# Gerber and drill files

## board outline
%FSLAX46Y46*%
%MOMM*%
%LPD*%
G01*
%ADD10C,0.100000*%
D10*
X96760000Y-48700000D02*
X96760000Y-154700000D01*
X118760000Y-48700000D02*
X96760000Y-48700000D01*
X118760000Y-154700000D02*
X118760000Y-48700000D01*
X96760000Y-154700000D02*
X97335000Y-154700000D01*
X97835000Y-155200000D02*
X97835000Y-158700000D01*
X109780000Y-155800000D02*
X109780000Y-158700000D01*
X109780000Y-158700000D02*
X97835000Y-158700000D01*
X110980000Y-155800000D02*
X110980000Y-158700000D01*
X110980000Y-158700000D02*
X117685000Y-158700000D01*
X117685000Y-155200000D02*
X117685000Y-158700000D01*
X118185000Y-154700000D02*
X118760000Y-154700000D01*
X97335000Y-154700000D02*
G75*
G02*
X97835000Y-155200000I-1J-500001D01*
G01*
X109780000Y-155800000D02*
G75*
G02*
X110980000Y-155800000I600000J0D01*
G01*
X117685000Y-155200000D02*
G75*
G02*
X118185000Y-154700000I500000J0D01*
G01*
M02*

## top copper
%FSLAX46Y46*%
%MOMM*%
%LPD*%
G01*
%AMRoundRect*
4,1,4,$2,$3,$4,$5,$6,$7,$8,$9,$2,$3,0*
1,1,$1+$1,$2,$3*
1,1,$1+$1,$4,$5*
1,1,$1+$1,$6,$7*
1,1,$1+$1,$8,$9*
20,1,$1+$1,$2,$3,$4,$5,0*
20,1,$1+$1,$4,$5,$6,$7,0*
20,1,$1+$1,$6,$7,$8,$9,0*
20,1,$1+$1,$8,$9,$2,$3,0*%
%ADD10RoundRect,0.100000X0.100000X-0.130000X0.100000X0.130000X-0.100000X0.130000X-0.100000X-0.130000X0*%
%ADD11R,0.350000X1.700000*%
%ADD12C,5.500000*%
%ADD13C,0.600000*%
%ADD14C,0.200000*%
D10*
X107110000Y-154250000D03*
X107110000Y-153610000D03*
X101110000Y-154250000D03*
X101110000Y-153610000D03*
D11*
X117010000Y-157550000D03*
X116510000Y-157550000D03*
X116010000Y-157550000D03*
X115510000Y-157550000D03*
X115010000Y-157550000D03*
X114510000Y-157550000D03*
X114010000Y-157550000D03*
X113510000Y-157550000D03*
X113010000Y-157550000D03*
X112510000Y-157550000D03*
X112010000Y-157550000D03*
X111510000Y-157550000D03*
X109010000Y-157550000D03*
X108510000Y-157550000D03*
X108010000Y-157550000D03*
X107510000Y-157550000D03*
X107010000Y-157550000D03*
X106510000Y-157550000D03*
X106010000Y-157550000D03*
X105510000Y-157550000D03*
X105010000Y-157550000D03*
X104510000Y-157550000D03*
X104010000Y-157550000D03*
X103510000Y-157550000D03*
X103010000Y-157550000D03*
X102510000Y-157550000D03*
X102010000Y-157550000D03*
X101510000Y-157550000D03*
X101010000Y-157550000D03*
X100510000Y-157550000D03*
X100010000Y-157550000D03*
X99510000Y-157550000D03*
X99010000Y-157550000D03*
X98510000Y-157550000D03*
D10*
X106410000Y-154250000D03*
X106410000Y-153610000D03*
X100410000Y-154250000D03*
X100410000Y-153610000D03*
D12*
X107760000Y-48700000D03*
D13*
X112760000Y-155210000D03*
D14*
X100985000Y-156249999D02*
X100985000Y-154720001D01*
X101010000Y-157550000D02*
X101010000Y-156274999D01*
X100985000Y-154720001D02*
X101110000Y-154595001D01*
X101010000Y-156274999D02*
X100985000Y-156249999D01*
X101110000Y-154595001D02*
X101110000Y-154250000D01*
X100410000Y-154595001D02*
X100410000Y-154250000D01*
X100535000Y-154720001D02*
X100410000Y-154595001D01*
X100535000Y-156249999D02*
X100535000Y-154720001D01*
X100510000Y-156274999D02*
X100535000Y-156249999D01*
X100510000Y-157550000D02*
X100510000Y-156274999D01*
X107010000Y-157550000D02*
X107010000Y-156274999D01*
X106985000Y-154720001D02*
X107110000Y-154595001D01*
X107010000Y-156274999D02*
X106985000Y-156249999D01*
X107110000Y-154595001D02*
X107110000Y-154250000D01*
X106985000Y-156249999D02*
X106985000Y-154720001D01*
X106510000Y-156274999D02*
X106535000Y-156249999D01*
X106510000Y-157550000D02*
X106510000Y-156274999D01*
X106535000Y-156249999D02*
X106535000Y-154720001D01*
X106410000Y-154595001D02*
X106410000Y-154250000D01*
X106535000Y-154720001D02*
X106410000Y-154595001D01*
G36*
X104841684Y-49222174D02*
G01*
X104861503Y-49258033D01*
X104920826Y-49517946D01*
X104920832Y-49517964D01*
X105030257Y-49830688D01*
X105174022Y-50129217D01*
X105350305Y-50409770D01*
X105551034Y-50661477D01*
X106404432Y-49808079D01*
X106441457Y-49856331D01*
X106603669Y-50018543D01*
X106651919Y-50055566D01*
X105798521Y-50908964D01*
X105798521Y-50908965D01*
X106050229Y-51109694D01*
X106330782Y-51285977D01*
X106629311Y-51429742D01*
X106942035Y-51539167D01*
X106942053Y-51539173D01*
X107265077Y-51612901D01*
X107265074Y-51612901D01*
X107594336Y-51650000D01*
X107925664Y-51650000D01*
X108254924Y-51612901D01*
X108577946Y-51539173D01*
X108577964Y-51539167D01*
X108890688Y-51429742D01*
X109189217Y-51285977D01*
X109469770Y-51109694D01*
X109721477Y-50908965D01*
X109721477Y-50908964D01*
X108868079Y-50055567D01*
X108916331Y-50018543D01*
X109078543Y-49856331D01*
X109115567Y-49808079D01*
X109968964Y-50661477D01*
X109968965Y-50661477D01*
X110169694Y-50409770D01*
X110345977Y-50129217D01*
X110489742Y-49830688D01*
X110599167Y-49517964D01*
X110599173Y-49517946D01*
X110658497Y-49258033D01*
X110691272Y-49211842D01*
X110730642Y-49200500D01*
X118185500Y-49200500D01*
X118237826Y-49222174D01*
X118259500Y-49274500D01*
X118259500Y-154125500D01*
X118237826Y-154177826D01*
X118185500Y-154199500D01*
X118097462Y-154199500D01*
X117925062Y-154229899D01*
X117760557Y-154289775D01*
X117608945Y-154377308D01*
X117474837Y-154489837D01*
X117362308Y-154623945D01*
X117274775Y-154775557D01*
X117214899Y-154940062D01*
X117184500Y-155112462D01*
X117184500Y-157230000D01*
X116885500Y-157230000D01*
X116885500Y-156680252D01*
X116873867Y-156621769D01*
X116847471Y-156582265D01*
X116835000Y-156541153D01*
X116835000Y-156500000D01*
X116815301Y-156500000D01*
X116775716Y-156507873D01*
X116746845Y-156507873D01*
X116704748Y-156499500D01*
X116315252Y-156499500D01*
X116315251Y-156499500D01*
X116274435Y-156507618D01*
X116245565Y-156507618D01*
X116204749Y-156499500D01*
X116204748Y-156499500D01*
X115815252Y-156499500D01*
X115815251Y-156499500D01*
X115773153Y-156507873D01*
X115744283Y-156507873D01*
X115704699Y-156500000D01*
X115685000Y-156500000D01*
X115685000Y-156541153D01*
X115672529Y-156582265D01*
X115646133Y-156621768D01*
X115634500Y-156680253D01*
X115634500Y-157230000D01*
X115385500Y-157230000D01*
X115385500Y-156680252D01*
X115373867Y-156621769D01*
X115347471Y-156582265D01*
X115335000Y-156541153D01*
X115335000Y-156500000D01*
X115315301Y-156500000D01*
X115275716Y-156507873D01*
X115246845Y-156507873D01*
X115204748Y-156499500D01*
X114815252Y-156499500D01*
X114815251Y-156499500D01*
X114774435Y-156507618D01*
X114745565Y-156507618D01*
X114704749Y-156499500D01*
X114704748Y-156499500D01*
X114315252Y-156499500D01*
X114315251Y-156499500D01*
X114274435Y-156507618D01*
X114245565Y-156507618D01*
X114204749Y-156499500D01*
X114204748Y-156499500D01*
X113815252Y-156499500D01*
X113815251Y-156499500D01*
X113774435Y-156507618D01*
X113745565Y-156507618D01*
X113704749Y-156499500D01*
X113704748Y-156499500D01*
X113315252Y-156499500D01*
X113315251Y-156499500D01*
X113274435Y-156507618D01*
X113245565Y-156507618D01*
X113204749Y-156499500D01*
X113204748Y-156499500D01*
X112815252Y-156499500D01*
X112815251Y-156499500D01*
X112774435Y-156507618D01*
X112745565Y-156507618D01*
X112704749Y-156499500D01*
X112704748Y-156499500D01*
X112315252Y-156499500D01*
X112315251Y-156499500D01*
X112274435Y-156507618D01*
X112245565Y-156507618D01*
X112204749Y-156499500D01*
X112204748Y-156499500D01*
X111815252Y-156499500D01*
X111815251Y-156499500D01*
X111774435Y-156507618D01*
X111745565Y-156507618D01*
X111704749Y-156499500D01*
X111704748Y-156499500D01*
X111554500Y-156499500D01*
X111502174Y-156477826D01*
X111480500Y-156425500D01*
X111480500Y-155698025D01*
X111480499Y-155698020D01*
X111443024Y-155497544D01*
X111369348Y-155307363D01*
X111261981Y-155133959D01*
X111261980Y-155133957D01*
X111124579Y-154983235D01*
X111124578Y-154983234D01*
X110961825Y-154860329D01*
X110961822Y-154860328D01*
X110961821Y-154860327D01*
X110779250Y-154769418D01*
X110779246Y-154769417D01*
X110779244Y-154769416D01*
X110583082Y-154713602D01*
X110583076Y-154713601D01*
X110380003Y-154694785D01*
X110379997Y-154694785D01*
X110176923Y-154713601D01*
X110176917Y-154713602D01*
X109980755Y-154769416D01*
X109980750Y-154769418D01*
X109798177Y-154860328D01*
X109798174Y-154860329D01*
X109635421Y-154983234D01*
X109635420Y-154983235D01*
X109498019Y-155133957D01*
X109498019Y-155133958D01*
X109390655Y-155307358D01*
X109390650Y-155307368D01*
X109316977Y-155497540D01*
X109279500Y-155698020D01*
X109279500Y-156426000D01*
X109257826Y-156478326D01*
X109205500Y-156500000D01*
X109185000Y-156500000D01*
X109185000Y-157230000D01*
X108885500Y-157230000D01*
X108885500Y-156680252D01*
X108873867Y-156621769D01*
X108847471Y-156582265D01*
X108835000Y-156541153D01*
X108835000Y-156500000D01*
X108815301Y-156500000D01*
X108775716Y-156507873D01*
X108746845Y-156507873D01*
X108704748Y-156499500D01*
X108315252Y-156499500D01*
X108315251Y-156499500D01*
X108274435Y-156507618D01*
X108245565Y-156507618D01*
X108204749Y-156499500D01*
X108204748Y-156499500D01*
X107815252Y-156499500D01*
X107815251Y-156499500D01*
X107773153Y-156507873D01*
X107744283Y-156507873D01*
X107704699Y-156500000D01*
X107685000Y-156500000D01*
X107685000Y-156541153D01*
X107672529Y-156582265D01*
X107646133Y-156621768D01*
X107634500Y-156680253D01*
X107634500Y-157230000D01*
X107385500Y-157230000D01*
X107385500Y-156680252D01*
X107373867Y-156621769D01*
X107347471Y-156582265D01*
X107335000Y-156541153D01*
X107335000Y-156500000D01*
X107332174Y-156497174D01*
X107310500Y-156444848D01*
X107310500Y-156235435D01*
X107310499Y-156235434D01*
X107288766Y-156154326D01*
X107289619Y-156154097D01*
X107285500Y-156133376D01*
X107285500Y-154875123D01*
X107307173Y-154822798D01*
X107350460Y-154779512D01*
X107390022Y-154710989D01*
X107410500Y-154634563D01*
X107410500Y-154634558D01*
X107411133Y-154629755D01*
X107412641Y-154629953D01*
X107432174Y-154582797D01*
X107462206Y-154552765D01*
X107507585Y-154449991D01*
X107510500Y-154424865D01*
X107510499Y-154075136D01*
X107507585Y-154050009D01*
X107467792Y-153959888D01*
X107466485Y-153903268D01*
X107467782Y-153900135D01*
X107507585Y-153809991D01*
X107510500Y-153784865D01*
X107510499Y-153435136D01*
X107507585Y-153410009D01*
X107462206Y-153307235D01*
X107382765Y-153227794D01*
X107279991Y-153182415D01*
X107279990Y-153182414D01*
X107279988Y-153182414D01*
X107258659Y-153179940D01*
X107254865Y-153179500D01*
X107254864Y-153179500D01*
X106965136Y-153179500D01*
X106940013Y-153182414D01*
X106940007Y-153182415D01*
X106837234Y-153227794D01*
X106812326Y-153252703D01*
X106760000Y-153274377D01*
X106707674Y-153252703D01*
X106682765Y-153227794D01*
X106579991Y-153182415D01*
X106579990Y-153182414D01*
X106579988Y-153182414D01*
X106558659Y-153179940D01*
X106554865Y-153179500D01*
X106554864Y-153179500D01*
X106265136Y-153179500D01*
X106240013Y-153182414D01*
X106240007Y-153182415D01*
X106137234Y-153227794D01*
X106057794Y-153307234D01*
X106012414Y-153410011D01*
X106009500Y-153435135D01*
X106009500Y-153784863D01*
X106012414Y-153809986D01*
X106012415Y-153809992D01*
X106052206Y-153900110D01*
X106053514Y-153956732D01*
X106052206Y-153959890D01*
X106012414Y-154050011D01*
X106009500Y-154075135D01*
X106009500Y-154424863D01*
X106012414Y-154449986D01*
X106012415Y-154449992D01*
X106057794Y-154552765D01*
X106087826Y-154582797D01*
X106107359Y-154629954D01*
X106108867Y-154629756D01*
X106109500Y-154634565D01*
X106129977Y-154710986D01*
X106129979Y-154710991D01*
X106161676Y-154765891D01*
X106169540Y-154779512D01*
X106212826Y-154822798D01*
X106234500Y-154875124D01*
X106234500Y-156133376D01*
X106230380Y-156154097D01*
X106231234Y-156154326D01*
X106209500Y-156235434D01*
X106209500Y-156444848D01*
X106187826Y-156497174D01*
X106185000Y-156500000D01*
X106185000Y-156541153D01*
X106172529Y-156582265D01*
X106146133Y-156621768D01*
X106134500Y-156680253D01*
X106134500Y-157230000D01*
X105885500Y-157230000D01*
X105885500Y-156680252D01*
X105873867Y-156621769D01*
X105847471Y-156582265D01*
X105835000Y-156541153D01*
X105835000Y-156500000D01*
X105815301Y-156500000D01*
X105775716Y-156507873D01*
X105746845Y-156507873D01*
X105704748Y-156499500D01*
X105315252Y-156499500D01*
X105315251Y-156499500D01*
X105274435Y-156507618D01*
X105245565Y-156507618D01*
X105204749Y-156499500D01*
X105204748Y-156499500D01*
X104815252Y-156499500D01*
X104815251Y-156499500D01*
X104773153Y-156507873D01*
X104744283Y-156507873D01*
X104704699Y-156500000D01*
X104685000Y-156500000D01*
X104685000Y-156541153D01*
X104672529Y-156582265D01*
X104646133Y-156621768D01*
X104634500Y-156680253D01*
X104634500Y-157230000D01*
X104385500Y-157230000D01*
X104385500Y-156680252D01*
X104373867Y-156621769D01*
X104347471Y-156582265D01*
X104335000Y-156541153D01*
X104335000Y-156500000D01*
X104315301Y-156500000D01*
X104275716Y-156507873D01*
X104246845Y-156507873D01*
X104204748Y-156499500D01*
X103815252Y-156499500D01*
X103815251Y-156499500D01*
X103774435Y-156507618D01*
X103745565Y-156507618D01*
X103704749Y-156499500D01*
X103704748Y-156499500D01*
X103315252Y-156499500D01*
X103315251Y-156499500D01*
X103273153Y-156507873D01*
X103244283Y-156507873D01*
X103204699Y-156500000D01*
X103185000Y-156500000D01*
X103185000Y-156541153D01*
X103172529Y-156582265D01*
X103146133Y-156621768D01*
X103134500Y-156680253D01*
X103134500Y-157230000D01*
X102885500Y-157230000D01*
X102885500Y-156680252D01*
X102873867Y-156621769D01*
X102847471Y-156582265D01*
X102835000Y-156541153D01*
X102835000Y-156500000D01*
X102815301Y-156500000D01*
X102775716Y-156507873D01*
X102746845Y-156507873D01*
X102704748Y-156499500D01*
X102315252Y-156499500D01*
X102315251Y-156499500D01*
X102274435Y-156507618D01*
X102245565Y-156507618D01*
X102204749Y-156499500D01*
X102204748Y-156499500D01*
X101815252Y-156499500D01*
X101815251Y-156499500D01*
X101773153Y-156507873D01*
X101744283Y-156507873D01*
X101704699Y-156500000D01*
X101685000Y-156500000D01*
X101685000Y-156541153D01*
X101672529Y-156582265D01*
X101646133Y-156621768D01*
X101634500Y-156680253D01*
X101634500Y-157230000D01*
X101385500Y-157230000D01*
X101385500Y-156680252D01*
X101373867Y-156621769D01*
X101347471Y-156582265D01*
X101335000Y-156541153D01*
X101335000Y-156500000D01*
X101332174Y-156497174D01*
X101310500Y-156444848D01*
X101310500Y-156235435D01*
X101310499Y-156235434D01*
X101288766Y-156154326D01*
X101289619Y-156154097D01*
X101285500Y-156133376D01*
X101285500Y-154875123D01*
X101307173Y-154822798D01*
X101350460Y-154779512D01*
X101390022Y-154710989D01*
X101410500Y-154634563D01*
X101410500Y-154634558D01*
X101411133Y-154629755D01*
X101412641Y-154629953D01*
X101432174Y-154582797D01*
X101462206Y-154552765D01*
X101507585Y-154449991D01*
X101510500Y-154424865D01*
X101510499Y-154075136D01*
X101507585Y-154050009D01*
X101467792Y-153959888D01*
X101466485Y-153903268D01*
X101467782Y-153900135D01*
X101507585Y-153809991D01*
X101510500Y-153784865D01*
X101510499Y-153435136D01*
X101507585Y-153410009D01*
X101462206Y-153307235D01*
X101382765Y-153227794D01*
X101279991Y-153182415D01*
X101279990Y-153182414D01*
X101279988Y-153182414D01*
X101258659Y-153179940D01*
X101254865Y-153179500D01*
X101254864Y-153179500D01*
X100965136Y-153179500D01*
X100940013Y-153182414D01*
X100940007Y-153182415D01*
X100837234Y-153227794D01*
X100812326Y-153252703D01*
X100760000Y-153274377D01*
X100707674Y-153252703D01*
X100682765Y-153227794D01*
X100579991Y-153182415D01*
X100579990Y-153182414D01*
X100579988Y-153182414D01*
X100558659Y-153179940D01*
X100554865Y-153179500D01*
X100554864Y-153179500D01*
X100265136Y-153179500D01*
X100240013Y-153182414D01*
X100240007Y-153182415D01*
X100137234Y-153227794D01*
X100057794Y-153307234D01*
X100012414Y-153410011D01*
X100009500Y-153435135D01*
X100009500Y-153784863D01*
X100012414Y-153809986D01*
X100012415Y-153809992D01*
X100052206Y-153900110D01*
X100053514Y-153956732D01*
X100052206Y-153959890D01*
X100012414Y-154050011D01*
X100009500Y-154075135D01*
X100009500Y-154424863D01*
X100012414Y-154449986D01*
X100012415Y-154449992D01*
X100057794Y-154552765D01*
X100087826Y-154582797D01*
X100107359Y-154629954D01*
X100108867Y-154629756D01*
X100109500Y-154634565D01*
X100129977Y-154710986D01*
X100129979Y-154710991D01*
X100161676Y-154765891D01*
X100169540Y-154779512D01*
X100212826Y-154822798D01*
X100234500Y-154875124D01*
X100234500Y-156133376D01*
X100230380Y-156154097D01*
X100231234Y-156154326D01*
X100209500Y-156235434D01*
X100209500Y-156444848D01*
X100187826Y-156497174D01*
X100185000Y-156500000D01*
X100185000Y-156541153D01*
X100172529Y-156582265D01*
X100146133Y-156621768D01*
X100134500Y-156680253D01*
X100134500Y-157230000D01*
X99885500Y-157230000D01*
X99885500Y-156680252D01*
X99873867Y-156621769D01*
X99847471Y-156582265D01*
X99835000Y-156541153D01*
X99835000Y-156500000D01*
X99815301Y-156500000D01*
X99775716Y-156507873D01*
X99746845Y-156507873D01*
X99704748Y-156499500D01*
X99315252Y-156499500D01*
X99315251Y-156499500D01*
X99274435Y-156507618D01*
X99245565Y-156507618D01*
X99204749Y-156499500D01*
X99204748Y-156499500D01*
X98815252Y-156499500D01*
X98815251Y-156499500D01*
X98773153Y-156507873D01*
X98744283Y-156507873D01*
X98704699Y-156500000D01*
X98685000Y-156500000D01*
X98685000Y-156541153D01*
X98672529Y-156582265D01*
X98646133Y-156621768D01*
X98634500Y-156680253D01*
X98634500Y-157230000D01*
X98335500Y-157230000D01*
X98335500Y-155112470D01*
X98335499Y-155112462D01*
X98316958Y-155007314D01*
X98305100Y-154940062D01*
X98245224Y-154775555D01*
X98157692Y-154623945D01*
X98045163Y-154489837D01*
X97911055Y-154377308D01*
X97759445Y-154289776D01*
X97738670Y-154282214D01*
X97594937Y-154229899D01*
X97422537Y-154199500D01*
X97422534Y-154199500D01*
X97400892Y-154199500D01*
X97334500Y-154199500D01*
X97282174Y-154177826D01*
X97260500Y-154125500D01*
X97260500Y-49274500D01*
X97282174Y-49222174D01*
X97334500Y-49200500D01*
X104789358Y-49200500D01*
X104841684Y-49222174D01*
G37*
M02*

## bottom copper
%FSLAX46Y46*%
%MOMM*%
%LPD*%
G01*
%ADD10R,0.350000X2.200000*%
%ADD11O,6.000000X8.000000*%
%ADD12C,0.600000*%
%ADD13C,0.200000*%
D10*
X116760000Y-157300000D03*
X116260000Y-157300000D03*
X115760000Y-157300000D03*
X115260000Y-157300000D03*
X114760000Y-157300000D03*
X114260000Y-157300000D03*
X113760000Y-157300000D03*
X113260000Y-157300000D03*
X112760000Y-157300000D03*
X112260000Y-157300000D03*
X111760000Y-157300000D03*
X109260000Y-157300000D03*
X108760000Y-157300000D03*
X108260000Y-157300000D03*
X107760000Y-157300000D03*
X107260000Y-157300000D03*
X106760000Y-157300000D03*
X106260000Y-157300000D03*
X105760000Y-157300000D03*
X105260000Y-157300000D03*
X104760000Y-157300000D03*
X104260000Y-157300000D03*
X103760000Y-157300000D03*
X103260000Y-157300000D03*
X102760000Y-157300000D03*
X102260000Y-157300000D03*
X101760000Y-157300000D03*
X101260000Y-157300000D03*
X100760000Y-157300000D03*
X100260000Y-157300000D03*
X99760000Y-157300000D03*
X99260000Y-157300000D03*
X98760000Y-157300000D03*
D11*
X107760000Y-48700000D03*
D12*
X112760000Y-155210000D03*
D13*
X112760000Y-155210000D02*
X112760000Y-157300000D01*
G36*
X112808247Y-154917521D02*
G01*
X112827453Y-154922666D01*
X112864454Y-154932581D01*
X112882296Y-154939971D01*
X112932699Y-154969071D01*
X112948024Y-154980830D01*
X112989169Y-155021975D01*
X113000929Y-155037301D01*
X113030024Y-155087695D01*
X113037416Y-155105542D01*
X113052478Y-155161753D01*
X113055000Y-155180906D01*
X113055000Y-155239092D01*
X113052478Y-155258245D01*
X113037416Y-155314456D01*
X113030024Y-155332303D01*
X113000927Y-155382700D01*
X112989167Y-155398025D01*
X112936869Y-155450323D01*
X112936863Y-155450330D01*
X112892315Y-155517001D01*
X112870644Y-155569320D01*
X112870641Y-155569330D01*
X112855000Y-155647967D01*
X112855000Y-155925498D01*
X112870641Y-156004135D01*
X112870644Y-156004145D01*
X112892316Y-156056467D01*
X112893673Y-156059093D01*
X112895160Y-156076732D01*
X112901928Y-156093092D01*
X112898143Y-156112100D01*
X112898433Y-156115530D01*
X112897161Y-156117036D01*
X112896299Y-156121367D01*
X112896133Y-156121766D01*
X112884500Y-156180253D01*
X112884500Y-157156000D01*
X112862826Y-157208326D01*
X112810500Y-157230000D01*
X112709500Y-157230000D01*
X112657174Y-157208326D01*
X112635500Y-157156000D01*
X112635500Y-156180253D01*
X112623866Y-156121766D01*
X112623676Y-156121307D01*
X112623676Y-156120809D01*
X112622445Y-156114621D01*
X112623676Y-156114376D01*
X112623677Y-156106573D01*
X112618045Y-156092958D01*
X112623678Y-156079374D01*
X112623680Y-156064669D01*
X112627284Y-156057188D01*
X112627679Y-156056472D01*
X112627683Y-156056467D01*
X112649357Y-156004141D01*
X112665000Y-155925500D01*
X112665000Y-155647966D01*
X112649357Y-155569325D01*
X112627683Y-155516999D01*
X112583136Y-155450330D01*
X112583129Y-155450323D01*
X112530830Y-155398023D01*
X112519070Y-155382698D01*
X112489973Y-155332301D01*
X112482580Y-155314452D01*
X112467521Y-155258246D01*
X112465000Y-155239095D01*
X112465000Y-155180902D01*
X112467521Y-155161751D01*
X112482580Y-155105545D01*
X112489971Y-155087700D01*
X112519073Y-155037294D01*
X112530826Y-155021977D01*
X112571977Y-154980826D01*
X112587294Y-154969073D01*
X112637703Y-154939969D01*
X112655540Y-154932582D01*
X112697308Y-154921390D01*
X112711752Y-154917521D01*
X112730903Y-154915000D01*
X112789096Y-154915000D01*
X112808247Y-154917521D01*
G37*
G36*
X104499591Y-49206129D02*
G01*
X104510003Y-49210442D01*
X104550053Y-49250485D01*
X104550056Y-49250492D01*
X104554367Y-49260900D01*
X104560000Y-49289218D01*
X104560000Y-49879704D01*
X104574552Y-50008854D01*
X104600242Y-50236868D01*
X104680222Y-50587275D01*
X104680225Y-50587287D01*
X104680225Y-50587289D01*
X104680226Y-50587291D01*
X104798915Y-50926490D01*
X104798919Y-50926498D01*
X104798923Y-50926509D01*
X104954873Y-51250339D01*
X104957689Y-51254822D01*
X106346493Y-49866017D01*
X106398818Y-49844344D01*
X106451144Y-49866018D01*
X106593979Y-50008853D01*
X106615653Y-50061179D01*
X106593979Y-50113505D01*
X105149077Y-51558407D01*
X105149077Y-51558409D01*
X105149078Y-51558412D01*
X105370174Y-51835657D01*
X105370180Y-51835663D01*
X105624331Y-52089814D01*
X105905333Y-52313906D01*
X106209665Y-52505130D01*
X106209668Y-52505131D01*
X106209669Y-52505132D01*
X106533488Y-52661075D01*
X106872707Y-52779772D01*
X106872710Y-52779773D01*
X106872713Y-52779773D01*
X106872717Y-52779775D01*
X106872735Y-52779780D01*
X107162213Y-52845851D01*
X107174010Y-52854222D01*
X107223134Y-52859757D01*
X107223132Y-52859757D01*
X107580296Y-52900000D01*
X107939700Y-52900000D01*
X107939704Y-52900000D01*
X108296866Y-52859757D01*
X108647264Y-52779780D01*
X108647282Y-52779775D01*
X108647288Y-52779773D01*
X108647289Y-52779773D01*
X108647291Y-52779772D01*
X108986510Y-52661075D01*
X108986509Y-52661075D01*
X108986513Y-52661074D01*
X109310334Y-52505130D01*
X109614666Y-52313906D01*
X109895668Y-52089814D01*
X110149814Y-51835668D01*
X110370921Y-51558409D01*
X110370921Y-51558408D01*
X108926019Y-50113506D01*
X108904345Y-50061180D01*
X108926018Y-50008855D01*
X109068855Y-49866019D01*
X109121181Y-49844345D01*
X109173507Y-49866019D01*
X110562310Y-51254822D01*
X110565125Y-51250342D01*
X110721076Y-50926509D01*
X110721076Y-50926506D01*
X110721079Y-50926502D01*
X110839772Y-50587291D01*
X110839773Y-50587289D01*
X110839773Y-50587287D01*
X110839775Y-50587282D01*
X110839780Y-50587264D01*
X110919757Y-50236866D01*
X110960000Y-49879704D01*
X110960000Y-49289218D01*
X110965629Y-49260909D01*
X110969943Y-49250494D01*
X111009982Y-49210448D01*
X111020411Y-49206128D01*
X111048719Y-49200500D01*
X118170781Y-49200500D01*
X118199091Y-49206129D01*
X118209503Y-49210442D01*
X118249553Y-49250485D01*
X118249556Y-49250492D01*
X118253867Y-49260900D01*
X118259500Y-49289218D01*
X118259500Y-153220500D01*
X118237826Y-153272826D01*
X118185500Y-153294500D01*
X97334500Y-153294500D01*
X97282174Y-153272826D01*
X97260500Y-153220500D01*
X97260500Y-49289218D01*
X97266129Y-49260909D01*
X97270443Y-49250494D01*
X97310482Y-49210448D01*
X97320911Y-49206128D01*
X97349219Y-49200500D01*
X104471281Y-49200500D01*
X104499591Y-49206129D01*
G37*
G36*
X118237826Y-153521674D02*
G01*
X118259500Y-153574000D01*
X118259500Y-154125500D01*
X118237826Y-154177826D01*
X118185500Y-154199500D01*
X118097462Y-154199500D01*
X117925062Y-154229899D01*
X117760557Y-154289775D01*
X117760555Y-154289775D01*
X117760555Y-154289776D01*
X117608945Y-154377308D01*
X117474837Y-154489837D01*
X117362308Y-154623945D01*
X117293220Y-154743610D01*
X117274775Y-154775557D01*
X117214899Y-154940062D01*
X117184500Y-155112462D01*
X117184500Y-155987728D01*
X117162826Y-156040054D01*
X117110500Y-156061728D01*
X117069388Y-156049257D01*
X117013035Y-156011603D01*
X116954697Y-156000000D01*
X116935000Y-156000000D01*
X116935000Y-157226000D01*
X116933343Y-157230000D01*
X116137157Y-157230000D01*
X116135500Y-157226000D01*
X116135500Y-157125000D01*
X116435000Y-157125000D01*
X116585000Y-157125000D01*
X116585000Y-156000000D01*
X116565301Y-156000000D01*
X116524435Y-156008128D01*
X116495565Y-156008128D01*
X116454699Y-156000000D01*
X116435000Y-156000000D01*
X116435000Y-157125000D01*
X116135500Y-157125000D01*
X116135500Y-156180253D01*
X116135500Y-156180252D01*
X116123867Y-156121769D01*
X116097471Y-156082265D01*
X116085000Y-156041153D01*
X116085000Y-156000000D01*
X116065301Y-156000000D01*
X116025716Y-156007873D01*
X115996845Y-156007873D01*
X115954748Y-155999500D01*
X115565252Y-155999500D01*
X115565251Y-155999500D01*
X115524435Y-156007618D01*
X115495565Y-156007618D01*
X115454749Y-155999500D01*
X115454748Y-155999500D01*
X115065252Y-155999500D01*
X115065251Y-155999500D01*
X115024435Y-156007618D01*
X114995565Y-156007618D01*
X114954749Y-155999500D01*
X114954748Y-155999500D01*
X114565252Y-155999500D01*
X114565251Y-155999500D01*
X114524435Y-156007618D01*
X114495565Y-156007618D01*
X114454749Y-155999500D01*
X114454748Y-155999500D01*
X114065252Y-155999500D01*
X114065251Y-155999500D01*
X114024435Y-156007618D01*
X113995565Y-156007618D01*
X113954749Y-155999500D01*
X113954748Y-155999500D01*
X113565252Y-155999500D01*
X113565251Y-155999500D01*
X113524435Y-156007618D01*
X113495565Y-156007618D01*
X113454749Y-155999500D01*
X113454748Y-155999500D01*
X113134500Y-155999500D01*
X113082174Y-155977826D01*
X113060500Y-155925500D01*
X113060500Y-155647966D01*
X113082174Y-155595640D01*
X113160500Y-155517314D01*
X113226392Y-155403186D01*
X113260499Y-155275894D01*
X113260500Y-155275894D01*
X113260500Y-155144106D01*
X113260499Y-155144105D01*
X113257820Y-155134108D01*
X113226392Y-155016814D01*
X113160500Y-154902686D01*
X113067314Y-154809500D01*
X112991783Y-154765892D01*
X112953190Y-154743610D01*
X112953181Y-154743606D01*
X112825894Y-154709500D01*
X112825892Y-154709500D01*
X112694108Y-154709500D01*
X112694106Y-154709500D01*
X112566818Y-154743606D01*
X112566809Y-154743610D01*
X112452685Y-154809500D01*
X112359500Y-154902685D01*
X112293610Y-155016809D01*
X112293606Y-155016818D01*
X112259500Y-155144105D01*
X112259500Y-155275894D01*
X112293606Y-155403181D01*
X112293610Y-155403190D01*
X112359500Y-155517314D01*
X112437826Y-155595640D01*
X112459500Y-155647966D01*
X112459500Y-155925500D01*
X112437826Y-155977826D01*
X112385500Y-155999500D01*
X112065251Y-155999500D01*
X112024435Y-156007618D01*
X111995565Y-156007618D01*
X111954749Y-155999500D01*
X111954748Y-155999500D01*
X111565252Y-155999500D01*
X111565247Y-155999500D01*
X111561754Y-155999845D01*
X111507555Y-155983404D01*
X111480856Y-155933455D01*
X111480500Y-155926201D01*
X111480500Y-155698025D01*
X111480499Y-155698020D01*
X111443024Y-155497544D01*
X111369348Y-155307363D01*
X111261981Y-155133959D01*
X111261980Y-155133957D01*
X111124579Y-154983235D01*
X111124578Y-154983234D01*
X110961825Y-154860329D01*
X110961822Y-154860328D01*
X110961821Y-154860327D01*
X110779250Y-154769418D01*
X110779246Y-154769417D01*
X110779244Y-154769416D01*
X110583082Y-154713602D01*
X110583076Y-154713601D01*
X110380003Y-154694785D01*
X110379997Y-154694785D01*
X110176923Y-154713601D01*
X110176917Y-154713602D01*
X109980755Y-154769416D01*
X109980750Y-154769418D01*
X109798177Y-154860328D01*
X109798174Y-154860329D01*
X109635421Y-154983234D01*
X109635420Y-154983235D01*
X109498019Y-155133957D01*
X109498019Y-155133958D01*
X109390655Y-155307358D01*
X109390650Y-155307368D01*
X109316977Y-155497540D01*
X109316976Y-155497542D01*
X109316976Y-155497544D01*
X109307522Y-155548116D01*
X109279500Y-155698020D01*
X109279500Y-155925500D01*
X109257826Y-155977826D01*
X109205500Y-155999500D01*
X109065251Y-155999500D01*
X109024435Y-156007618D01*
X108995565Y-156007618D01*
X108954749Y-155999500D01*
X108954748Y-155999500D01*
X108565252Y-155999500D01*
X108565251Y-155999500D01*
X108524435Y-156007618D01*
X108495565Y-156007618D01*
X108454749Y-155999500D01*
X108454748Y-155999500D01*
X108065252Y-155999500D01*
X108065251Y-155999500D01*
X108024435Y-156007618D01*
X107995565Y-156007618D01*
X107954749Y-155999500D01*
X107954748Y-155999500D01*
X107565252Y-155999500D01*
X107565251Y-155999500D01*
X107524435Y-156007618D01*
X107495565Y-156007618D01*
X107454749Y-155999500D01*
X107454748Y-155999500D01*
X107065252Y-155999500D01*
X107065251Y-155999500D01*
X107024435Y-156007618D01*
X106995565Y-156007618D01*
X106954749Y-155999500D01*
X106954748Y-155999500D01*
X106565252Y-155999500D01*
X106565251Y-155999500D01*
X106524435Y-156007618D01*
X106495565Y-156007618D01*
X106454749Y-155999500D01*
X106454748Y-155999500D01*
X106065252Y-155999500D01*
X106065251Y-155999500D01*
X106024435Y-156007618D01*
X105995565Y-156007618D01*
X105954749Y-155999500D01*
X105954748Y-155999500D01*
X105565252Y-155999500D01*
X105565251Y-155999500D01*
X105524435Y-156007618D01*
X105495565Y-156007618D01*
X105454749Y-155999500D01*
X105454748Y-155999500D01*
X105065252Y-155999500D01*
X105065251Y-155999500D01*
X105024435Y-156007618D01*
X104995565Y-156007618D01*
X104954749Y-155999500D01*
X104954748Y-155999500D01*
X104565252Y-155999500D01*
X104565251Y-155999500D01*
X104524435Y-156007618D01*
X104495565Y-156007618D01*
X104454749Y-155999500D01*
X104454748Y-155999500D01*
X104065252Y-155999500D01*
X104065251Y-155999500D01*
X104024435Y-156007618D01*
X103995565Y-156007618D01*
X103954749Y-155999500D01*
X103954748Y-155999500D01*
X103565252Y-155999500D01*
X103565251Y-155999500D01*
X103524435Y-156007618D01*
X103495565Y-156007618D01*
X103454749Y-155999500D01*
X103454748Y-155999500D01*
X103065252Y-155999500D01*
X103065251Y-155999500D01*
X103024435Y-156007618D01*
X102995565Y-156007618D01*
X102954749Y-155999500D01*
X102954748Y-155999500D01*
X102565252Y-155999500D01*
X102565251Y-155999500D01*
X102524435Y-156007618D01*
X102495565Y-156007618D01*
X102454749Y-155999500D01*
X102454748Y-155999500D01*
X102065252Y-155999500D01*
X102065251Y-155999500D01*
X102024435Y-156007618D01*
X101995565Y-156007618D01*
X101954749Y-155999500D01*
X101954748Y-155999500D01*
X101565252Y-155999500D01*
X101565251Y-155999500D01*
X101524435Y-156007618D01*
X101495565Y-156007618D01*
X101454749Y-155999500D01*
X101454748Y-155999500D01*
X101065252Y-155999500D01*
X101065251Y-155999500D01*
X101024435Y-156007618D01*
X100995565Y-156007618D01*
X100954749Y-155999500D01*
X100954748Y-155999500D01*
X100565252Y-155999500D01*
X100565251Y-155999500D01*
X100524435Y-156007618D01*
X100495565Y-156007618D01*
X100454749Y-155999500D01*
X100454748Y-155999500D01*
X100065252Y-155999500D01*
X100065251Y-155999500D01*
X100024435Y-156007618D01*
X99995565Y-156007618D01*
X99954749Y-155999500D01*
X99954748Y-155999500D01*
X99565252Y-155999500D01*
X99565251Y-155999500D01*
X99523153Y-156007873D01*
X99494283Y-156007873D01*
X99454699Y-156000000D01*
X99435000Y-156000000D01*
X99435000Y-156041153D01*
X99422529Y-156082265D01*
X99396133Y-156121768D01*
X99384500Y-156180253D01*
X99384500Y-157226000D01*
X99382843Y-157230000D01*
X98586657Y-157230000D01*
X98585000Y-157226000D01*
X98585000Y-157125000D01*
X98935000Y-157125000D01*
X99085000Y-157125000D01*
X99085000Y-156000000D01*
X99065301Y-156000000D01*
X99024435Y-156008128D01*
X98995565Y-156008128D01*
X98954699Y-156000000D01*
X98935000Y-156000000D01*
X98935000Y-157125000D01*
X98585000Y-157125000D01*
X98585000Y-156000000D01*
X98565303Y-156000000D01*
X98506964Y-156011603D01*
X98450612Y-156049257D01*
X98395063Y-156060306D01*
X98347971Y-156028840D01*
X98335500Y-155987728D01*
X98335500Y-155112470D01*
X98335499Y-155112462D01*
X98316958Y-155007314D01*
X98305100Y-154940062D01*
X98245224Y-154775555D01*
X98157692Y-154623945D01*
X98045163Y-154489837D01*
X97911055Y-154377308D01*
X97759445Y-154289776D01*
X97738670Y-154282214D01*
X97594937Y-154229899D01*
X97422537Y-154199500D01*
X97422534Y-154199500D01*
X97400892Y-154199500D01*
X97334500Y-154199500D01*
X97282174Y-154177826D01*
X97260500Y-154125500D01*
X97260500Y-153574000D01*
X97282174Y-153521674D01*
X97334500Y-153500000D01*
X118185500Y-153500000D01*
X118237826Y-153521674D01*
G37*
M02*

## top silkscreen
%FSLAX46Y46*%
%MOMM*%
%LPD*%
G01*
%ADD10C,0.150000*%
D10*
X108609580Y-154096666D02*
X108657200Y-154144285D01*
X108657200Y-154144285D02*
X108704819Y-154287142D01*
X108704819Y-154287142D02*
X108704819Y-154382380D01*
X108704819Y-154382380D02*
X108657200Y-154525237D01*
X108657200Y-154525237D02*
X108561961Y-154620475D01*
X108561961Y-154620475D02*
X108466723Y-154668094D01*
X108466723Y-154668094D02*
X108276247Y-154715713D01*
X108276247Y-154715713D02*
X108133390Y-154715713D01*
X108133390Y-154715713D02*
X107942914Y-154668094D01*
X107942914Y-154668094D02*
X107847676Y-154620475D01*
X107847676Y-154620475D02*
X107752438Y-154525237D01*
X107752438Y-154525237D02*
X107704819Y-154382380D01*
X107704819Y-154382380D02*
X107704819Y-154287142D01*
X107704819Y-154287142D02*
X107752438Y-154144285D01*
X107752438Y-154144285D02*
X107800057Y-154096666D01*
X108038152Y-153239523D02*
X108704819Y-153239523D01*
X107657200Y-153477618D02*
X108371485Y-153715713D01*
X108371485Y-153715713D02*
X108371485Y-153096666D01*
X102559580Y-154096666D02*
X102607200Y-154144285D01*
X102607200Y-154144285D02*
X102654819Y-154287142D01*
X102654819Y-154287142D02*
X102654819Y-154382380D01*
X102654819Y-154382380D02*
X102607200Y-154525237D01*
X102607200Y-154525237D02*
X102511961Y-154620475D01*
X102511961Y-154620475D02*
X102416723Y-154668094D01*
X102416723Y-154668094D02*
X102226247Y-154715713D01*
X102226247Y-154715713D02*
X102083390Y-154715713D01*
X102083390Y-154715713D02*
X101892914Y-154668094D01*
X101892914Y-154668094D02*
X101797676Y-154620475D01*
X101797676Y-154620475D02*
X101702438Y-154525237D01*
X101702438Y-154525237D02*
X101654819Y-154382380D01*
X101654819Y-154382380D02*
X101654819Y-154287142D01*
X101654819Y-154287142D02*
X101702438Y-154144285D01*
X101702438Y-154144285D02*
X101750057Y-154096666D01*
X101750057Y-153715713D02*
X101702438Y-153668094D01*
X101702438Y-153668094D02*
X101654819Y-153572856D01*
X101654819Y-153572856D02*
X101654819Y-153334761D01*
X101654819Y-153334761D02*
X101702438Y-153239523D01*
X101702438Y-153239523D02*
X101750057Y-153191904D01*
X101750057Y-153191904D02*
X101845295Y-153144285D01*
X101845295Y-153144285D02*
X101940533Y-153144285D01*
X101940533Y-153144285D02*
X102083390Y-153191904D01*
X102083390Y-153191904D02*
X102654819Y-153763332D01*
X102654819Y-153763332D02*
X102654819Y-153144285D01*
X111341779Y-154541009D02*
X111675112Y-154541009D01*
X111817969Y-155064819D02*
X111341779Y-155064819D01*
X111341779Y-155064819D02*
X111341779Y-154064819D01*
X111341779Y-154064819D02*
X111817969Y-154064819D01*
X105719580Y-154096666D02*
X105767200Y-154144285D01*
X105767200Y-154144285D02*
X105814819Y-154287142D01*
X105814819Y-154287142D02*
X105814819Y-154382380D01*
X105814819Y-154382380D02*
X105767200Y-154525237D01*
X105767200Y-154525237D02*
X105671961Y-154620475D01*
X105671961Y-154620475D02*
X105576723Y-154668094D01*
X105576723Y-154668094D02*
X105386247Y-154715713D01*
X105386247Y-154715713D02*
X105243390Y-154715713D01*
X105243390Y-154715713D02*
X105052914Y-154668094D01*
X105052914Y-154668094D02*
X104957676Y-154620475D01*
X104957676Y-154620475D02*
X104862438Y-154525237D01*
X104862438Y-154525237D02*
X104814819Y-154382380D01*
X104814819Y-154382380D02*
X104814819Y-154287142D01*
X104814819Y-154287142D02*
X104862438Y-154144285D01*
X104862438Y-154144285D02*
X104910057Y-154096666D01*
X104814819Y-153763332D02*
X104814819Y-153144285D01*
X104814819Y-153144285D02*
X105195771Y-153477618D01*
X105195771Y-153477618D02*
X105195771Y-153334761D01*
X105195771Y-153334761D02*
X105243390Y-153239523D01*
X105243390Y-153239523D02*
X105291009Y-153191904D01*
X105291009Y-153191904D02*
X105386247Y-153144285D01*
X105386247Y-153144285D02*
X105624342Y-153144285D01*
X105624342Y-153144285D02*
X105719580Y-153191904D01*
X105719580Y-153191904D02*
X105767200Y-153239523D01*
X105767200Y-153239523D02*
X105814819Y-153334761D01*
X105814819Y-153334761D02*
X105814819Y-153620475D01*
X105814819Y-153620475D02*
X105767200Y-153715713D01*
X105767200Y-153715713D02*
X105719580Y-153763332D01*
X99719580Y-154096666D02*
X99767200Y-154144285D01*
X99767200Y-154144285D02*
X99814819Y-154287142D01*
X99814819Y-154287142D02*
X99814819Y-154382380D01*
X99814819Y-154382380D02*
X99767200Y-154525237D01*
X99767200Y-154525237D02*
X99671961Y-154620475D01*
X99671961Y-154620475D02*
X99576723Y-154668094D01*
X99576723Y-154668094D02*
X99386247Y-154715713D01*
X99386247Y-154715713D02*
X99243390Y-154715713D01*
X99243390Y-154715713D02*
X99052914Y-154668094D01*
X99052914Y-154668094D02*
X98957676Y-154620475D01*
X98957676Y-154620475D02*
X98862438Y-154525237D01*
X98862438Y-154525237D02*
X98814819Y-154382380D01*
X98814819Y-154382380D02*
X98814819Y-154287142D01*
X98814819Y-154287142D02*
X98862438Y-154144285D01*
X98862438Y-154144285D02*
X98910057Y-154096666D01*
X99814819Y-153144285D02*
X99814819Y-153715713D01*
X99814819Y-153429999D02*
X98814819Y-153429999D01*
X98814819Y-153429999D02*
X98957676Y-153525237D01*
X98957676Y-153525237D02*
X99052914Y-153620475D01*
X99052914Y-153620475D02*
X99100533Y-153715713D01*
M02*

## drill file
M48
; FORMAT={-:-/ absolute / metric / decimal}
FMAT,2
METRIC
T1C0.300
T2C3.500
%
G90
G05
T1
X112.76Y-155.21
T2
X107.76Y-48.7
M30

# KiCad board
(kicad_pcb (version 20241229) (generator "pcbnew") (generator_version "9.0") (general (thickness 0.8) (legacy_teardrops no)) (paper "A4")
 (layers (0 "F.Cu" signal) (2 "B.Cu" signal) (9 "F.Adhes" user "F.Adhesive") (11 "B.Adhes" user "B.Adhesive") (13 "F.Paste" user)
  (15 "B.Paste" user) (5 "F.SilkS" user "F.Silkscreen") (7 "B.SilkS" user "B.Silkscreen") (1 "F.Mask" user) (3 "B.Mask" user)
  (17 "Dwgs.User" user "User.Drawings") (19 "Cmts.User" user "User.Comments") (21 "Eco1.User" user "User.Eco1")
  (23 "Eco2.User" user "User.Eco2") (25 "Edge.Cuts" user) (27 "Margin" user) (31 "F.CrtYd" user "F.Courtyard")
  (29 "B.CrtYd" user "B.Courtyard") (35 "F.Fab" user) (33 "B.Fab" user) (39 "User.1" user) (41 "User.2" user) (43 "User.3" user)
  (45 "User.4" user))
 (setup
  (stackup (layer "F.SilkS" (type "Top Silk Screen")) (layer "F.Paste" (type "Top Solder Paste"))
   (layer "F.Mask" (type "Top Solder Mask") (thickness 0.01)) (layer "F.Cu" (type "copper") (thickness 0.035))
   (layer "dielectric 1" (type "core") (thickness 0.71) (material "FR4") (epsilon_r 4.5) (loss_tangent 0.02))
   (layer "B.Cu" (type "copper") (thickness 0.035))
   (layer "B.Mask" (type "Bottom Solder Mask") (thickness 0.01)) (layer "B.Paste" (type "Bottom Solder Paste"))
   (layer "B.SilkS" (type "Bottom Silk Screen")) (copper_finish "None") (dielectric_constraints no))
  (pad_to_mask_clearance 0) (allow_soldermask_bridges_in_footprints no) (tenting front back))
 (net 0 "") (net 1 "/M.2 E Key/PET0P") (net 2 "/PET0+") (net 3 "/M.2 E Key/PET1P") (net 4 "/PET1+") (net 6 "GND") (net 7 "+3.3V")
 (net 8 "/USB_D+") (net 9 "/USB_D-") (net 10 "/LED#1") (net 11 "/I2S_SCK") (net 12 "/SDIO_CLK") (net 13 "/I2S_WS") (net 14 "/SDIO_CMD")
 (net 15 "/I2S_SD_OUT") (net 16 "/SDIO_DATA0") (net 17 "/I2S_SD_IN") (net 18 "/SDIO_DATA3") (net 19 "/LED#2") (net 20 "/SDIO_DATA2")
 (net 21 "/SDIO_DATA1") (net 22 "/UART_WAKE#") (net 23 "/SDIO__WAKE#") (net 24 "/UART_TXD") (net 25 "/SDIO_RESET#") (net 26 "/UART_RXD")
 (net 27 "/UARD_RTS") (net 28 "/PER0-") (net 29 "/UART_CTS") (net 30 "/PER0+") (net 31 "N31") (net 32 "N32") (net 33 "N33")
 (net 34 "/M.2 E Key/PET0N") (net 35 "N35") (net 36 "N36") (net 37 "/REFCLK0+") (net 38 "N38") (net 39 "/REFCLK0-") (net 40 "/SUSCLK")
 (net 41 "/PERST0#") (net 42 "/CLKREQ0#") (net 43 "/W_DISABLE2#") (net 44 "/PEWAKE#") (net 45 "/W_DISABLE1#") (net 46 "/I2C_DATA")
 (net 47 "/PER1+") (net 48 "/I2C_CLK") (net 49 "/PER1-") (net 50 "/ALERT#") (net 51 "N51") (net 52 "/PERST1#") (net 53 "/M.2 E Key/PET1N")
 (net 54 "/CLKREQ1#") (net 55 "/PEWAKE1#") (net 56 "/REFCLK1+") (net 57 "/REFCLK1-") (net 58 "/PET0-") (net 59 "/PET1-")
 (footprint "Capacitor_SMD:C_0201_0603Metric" (layer "F.Cu") (at 107.11 153.93 90)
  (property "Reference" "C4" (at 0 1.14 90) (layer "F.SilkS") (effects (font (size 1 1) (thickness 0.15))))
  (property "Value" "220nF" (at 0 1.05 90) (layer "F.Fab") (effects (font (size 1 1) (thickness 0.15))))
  (pad "" smd roundrect (at -0.345 0 90) (size 0.318 0.36) (layers "F.Paste") (roundrect_rratio 0.25))
  (pad "" smd roundrect (at 0.345 0 90) (size 0.318 0.36) (layers "F.Paste") (roundrect_rratio 0.25))
  (pad "1" smd roundrect (at -0.32 0 90) (size 0.46 0.4) (layers "F.Cu" "F.Mask") (roundrect_rratio 0.25) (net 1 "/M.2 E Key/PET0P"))
  (pad "2" smd roundrect (at 0.32 0 90) (size 0.46 0.4) (layers "F.Cu" "F.Mask") (roundrect_rratio 0.25) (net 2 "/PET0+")))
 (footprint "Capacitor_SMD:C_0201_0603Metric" (layer "F.Cu") (at 101.11 153.93 90)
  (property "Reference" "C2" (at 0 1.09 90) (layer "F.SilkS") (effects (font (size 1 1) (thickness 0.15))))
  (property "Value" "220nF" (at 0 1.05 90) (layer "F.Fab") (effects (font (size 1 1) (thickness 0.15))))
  (pad "" smd roundrect (at -0.345 0 90) (size 0.318 0.36) (layers "F.Paste") (roundrect_rratio 0.25))
  (pad "" smd roundrect (at 0.345 0 90) (size 0.318 0.36) (layers "F.Paste") (roundrect_rratio 0.25))
  (pad "1" smd roundrect (at -0.32 0 90) (size 0.46 0.4) (layers "F.Cu" "F.Mask") (roundrect_rratio 0.25) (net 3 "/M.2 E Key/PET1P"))
  (pad "2" smd roundrect (at 0.32 0 90) (size 0.46 0.4) (layers "F.Cu" "F.Mask") (roundrect_rratio 0.25) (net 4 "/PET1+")))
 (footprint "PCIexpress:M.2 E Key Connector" (layer "F.Cu") (at 107.76 157.59)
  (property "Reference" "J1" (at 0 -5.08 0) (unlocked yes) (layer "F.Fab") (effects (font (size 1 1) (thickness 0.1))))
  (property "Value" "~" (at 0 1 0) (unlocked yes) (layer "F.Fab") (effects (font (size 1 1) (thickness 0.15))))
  (fp_line (start -11 -2.89) (end -10.425 -2.89) (stroke (width 0.1) (type default)) (layer "Edge.Cuts") (net 5))
  (fp_line (start -9.925 -2.39) (end -9.925 1.11) (stroke (width 0.1) (type default)) (layer "Edge.Cuts") (net 5))
  (fp_line (start 2.02 -1.79) (end 2.02 1.11) (stroke (width 0.1) (type default)) (layer "Edge.Cuts") (net 5))
  (fp_line (start 2.02 1.11) (end -9.925 1.11) (stroke (width 0.1) (type default)) (layer "Edge.Cuts") (net 5))
  (fp_line (start 3.22 -1.79) (end 3.22 1.11) (stroke (width 0.1) (type default)) (layer "Edge.Cuts") (net 5))
  (fp_line (start 3.22 1.11) (end 9.925 1.11) (stroke (width 0.1) (type default)) (layer "Edge.Cuts") (net 5))
  (fp_line (start 9.925 -2.39) (end 9.925 1.11) (stroke (width 0.1) (type default)) (layer "Edge.Cuts") (net 5))
  (fp_line (start 10.425 -2.89) (end 11 -2.89) (stroke (width 0.1) (type default)) (layer "Edge.Cuts") (net 5))
  (fp_arc (start -10.425 -2.89) (mid -10.071447 -2.743553) (end -9.925 -2.39) (stroke (width 0.1) (type default)) (layer "Edge.Cuts")
   (net 5))
  (fp_arc (start 2.02 -1.79) (mid 2.62 -2.39) (end 3.22 -1.79) (stroke (width 0.1) (type default)) (layer "Edge.Cuts") (net 5))
  (fp_arc (start 9.925 -2.39) (mid 10.071447 -2.743553) (end 10.425 -2.89) (stroke (width 0.1) (type default)) (layer "Edge.Cuts") (net 5))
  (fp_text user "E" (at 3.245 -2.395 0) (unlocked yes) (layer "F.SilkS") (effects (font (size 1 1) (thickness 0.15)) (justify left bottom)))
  (pad "1" smd rect (at 9.25 -0.04 180) (size 0.35 1.7) (layers "F.Cu") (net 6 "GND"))
  (pad "2" smd rect (at 9 -0.29 180) (size 0.35 2.2) (layers "B.Cu") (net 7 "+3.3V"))
  (pad "3" smd rect (at 8.75 -0.04 180) (size 0.35 1.7) (layers "F.Cu") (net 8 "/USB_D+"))
  (pad "4" smd rect (at 8.5 -0.29 180) (size 0.35 2.2) (layers "B.Cu") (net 7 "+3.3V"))
  (pad "5" smd rect (at 8.25 -0.04 180) (size 0.35 1.7) (layers "F.Cu") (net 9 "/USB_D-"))
  (pad "6" smd rect (at 8 -0.29 180) (size 0.35 2.2) (layers "B.Cu") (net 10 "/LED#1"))
  (pad "7" smd rect (at 7.75 -0.04 180) (size 0.35 1.7) (layers "F.Cu") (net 6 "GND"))
  (pad "8" smd rect (at 7.5 -0.29 180) (size 0.35 2.2) (layers "B.Cu") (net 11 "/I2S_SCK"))
  (pad "9" smd rect (at 7.25 -0.04 180) (size 0.35 1.7) (layers "F.Cu") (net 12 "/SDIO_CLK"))
  (pad "10" smd rect (at 7 -0.29 180) (size 0.35 2.2) (layers "B.Cu") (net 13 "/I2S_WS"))
  (pad "11" smd rect (at 6.75 -0.04 180) (size 0.35 1.7) (layers "F.Cu") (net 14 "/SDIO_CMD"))
  (pad "12" smd rect (at 6.5 -0.29 180) (size 0.35 2.2) (layers "B.Cu") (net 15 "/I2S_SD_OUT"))
  (pad "13" smd rect (at 6.25 -0.04 180) (size 0.35 1.7) (layers "F.Cu") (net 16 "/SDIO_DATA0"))
  (pad "14" smd rect (at 6 -0.29 180) (size 0.35 2.2) (layers "B.Cu") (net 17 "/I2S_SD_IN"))
  (pad "15" smd rect (at 5.75 -0.04 180) (size 0.35 1.7) (layers "F.Cu") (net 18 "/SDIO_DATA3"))
  (pad "16" smd rect (at 5.5 -0.29 180) (size 0.35 2.2) (layers "B.Cu") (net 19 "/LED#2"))
  (pad "17" smd rect (at 5.25 -0.04 180) (size 0.35 1.7) (layers "F.Cu") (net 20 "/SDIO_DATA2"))
  (pad "18" smd rect (at 5 -0.29 180) (size 0.35 2.2) (layers "B.Cu") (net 6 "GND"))
  (pad "19" smd rect (at 4.75 -0.04 180) (size 0.35 1.7) (layers "F.Cu") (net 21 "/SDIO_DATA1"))
  (pad "20" smd rect (at 4.5 -0.29 180) (size 0.35 2.2) (layers "B.Cu") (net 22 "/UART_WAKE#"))
  (pad "21" smd rect (at 4.25 -0.04 180) (size 0.35 1.7) (layers "F.Cu") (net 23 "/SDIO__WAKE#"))
  (pad "22" smd rect (at 4 -0.29 180) (size 0.35 2.2) (layers "B.Cu") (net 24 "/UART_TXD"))
  (pad "23" smd rect (at 3.75 -0.04 180) (size 0.35 1.7) (layers "F.Cu") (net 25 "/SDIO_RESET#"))
  (pad "32" smd rect (at 1.5 -0.29 180) (size 0.35 2.2) (layers "B.Cu") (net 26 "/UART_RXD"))
  (pad "33" smd rect (at 1.25 -0.04 180) (size 0.35 1.7) (layers "F.Cu") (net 6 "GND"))
  (pad "34" smd rect (at 1 -0.29 180) (size 0.35 2.2) (layers "B.Cu") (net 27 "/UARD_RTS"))
  (pad "35" smd rect (at 0.75 -0.04 180) (size 0.35 1.7) (layers "F.Cu") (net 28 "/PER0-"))
  (pad "36" smd rect (at 0.5 -0.29 180) (size 0.35 2.2) (layers "B.Cu") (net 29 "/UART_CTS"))
  (pad "37" smd rect (at 0.25 -0.04 180) (size 0.35 1.7) (layers "F.Cu") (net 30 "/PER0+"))
  (pad "38" smd rect (at 0 -0.29 180) (size 0.35 2.2) (layers "B.Cu") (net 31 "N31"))
  (pad "39" smd rect (at -0.25 -0.04 180) (size 0.35 1.7) (layers "F.Cu") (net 6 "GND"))
  (pad "40" smd rect (at -0.5 -0.29 180) (size 0.35 2.2) (layers "B.Cu") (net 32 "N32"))
  (pad "41" smd rect (at -0.75 -0.04 180) (size 0.35 1.7) (layers "F.Cu") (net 1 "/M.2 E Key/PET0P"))
  (pad "42" smd rect (at -1 -0.29 180) (size 0.35 2.2) (layers "B.Cu") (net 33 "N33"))
  (pad "43" smd rect (at -1.25 -0.04 180) (size 0.35 1.7) (layers "F.Cu") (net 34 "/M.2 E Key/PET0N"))
  (pad "44" smd rect (at -1.5 -0.29 180) (size 0.35 2.2) (layers "B.Cu") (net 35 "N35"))
  (pad "45" smd rect (at -1.75 -0.04 180) (size 0.35 1.7) (layers "F.Cu") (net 6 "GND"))
  (pad "46" smd rect (at -2 -0.29 180) (size 0.35 2.2) (layers "B.Cu") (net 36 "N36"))
  (pad "47" smd rect (at -2.25 -0.04 180) (size 0.35 1.7) (layers "F.Cu") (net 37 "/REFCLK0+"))
  (pad "48" smd rect (at -2.5 -0.29 180) (size 0.35 2.2) (layers "B.Cu") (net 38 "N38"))
  (pad "49" smd rect (at -2.75 -0.04 180) (size 0.35 1.7) (layers "F.Cu") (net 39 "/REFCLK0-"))
  (pad "50" smd rect (at -3 -0.29 180) (size 0.35 2.2) (layers "B.Cu") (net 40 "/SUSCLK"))
  (pad "51" smd rect (at -3.25 -0.04 180) (size 0.35 1.7) (layers "F.Cu") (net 6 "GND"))
  (pad "52" smd rect (at -3.5 -0.29 180) (size 0.35 2.2) (layers "B.Cu") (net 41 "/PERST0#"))
  (pad "53" smd rect (at -3.75 -0.04 180) (size 0.35 1.7) (layers "F.Cu") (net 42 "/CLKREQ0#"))
  (pad "54" smd rect (at -4 -0.29 180) (size 0.35 2.2) (layers "B.Cu") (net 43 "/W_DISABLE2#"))
  (pad "55" smd rect (at -4.25 -0.04 180) (size 0.35 1.7) (layers "F.Cu") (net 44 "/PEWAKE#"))
  (pad "56" smd rect (at -4.5 -0.29 180) (size 0.35 2.2) (layers "B.Cu") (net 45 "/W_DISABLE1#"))
  (pad "57" smd rect (at -4.75 -0.04 180) (size 0.35 1.7) (layers "F.Cu") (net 6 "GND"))
  (pad "58" smd rect (at -5 -0.29 180) (size 0.35 2.2) (layers "B.Cu") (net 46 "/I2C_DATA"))
  (pad "59" smd rect (at -5.25 -0.04 180) (size 0.35 1.7) (layers "F.Cu") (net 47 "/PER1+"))
  (pad "60" smd rect (at -5.5 -0.29 180) (size 0.35 2.2) (layers "B.Cu") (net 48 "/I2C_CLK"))
  (pad "61" smd rect (at -5.75 -0.04 180) (size 0.35 1.7) (layers "F.Cu") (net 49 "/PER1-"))
  (pad "62" smd rect (at -6 -0.29 180) (size 0.35 2.2) (layers "B.Cu") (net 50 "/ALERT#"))
  (pad "63" smd rect (at -6.25 -0.04 180) (size 0.35 1.7) (layers "F.Cu") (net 6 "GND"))
  (pad "64" smd rect (at -6.5 -0.29 180) (size 0.35 2.2) (layers "B.Cu") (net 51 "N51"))
  (pad "65" smd rect (at -6.75 -0.04 180) (size 0.35 1.7) (layers "F.Cu") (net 3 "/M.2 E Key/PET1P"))
  (pad "66" smd rect (at -7 -0.29 180) (size 0.35 2.2) (layers "B.Cu") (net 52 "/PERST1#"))
  (pad "67" smd rect (at -7.25 -0.04 180) (size 0.35 1.7) (layers "F.Cu") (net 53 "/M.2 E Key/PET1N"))
  (pad "68" smd rect (at -7.5 -0.29 180) (size 0.35 2.2) (layers "B.Cu") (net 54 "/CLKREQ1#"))
  (pad "69" smd rect (at -7.75 -0.04 180) (size 0.35 1.7) (layers "F.Cu") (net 6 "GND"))
  (pad "70" smd rect (at -8 -0.29 180) (size 0.35 2.2) (layers "B.Cu") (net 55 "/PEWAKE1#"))
  (pad "71" smd rect (at -8.25 -0.04 180) (size 0.35 1.7) (layers "F.Cu") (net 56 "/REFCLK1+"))
  (pad "72" smd rect (at -8.5 -0.29 180) (size 0.35 2.2) (layers "B.Cu") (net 7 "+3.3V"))
  (pad "73" smd rect (at -8.75 -0.04 180) (size 0.35 1.7) (layers "F.Cu") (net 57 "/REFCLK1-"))
  (pad "74" smd rect (at -9 -0.29 180) (size 0.35 2.2) (layers "B.Cu") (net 7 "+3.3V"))
  (pad "75" smd rect (at -9.25 -0.04 180) (size 0.35 1.7) (layers "F.Cu") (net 6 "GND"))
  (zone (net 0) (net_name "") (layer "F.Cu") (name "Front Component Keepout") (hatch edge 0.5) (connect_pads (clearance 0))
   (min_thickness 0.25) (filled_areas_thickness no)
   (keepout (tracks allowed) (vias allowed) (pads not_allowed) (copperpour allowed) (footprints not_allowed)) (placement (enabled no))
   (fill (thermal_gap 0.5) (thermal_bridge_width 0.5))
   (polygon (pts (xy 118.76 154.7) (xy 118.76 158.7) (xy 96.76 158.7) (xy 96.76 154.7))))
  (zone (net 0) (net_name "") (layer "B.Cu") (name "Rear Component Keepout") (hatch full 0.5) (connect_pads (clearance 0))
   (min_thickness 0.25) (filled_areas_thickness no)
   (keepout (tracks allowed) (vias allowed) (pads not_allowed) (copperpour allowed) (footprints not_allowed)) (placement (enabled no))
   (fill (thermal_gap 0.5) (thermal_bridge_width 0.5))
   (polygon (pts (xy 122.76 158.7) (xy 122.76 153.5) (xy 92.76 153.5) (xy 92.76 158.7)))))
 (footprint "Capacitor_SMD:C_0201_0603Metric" (layer "F.Cu") (at 106.41 153.93 90)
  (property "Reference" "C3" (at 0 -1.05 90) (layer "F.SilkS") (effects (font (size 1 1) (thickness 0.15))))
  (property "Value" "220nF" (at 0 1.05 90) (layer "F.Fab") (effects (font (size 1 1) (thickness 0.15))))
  (pad "" smd roundrect (at -0.345 0 90) (size 0.318 0.36) (layers "F.Paste") (roundrect_rratio 0.25))
  (pad "" smd roundrect (at 0.345 0 90) (size 0.318 0.36) (layers "F.Paste") (roundrect_rratio 0.25))
  (pad "1" smd roundrect (at -0.32 0 90) (size 0.46 0.4) (layers "F.Cu" "F.Mask") (roundrect_rratio 0.25) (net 34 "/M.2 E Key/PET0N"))
  (pad "2" smd roundrect (at 0.32 0 90) (size 0.46 0.4) (layers "F.Cu" "F.Mask") (roundrect_rratio 0.25) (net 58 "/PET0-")))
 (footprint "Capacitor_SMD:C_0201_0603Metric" (layer "F.Cu") (at 100.41 153.93 90)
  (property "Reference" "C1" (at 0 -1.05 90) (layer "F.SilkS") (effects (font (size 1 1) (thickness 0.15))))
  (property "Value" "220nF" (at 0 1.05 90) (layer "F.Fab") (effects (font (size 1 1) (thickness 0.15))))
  (pad "" smd roundrect (at -0.345 0 90) (size 0.318 0.36) (layers "F.Paste") (roundrect_rratio 0.25))
  (pad "" smd roundrect (at 0.345 0 90) (size 0.318 0.36) (layers "F.Paste") (roundrect_rratio 0.25))
  (pad "1" smd roundrect (at -0.32 0 90) (size 0.46 0.4) (layers "F.Cu" "F.Mask") (roundrect_rratio 0.25) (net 53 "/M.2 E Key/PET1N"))
  (pad "2" smd roundrect (at 0.32 0 90) (size 0.46 0.4) (layers "F.Cu" "F.Mask") (roundrect_rratio 0.25) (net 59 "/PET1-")))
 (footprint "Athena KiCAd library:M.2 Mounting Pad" (layer "F.Cu") (at 107.76 48.7)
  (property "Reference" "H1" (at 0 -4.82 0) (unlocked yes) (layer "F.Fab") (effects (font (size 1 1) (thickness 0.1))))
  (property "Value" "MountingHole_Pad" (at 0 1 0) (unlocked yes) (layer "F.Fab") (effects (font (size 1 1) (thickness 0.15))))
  (pad "1" thru_hole circle (at 0 0) (size 5.5 5.5) (drill 3.5) (layers "*.Cu" "*.Mask") (remove_unused_layers no) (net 6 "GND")
   (padstack (mode front_inner_back)
    (layer "Inner" (shape circle) (size 5.5 5.5) (zone_connect -1))
    (layer "B.Cu" (shape oval) (size 6 8) (thermal_bridge_angle 45) (zone_connect -1)))))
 (gr_line (start 96.76 48.7) (end 96.76 154.7) (stroke (width 0.1) (type default)) (layer "Edge.Cuts"))
 (gr_line (start 118.76 48.7) (end 96.76 48.7) (stroke (width 0.1) (type default)) (layer "Edge.Cuts"))
 (gr_line (start 118.76 154.7) (end 118.76 48.7) (stroke (width 0.1) (type default)) (layer "Edge.Cuts"))
 (segment (start 100.985 156.249999) (end 100.985 154.720001) (width 0.2) (layer "F.Cu") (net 3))
 (segment (start 101.01 157.55) (end 101.01 156.274999) (width 0.2) (layer "F.Cu") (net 3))
 (segment (start 100.985 154.720001) (end 101.11 154.595001) (width 0.2) (layer "F.Cu") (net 3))
 (segment (start 101.01 156.274999) (end 100.985 156.249999) (width 0.2) (layer "F.Cu") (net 3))
 (segment (start 101.11 154.595001) (end 101.11 154.25) (width 0.2) (layer "F.Cu") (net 3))
 (segment (start 100.41 154.595001) (end 100.41 154.25) (width 0.2) (layer "F.Cu") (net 53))
 (segment (start 100.535 154.720001) (end 100.41 154.595001) (width 0.2) (layer "F.Cu") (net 53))
 (segment (start 100.535 156.249999) (end 100.535 154.720001) (width 0.2) (layer "F.Cu") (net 53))
 (segment (start 100.51 156.274999) (end 100.535 156.249999) (width 0.2) (layer "F.Cu") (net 53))
 (segment (start 100.51 157.55) (end 100.51 156.274999) (width 0.2) (layer "F.Cu") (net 53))
 (segment (start 107.01 157.55) (end 107.01 156.274999) (width 0.2) (layer "F.Cu") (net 1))
 (segment (start 106.985 154.720001) (end 107.11 154.595001) (width 0.2) (layer "F.Cu") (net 1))
 (segment (start 107.01 156.274999) (end 106.985 156.249999) (width 0.2) (layer "F.Cu") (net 1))
 (segment (start 107.11 154.595001) (end 107.11 154.25) (width 0.2) (layer "F.Cu") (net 1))
 (segment (start 106.985 156.249999) (end 106.985 154.720001) (width 0.2) (layer "F.Cu") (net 1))
 (segment (start 106.51 156.274999) (end 106.535 156.249999) (width 0.2) (layer "F.Cu") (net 34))
 (segment (start 106.51 157.55) (end 106.51 156.274999) (width 0.2) (layer "F.Cu") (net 34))
 (segment (start 106.535 156.249999) (end 106.535 154.720001) (width 0.2) (layer "F.Cu") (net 34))
 (segment (start 106.41 154.595001) (end 106.41 154.25) (width 0.2) (layer "F.Cu") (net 34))
 (segment (start 106.535 154.720001) (end 106.41 154.595001) (width 0.2) (layer "F.Cu") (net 34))
 (via (at 112.76 155.21) (size 0.6) (drill 0.3) (layers "F.Cu" "B.Cu") (free yes) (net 6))
 (segment (start 112.76 155.21) (end 112.76 157.3) (width 0.2) (layer "B.Cu") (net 6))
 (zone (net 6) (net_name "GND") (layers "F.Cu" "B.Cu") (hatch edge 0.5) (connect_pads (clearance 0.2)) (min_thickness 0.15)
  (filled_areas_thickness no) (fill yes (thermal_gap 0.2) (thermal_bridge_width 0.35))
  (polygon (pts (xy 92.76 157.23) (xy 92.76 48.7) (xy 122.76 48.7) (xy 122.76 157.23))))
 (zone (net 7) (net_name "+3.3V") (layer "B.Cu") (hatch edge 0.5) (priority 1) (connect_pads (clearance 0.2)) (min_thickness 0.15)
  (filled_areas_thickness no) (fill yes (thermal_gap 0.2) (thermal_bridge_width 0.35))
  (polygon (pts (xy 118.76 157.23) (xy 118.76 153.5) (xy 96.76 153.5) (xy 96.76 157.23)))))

